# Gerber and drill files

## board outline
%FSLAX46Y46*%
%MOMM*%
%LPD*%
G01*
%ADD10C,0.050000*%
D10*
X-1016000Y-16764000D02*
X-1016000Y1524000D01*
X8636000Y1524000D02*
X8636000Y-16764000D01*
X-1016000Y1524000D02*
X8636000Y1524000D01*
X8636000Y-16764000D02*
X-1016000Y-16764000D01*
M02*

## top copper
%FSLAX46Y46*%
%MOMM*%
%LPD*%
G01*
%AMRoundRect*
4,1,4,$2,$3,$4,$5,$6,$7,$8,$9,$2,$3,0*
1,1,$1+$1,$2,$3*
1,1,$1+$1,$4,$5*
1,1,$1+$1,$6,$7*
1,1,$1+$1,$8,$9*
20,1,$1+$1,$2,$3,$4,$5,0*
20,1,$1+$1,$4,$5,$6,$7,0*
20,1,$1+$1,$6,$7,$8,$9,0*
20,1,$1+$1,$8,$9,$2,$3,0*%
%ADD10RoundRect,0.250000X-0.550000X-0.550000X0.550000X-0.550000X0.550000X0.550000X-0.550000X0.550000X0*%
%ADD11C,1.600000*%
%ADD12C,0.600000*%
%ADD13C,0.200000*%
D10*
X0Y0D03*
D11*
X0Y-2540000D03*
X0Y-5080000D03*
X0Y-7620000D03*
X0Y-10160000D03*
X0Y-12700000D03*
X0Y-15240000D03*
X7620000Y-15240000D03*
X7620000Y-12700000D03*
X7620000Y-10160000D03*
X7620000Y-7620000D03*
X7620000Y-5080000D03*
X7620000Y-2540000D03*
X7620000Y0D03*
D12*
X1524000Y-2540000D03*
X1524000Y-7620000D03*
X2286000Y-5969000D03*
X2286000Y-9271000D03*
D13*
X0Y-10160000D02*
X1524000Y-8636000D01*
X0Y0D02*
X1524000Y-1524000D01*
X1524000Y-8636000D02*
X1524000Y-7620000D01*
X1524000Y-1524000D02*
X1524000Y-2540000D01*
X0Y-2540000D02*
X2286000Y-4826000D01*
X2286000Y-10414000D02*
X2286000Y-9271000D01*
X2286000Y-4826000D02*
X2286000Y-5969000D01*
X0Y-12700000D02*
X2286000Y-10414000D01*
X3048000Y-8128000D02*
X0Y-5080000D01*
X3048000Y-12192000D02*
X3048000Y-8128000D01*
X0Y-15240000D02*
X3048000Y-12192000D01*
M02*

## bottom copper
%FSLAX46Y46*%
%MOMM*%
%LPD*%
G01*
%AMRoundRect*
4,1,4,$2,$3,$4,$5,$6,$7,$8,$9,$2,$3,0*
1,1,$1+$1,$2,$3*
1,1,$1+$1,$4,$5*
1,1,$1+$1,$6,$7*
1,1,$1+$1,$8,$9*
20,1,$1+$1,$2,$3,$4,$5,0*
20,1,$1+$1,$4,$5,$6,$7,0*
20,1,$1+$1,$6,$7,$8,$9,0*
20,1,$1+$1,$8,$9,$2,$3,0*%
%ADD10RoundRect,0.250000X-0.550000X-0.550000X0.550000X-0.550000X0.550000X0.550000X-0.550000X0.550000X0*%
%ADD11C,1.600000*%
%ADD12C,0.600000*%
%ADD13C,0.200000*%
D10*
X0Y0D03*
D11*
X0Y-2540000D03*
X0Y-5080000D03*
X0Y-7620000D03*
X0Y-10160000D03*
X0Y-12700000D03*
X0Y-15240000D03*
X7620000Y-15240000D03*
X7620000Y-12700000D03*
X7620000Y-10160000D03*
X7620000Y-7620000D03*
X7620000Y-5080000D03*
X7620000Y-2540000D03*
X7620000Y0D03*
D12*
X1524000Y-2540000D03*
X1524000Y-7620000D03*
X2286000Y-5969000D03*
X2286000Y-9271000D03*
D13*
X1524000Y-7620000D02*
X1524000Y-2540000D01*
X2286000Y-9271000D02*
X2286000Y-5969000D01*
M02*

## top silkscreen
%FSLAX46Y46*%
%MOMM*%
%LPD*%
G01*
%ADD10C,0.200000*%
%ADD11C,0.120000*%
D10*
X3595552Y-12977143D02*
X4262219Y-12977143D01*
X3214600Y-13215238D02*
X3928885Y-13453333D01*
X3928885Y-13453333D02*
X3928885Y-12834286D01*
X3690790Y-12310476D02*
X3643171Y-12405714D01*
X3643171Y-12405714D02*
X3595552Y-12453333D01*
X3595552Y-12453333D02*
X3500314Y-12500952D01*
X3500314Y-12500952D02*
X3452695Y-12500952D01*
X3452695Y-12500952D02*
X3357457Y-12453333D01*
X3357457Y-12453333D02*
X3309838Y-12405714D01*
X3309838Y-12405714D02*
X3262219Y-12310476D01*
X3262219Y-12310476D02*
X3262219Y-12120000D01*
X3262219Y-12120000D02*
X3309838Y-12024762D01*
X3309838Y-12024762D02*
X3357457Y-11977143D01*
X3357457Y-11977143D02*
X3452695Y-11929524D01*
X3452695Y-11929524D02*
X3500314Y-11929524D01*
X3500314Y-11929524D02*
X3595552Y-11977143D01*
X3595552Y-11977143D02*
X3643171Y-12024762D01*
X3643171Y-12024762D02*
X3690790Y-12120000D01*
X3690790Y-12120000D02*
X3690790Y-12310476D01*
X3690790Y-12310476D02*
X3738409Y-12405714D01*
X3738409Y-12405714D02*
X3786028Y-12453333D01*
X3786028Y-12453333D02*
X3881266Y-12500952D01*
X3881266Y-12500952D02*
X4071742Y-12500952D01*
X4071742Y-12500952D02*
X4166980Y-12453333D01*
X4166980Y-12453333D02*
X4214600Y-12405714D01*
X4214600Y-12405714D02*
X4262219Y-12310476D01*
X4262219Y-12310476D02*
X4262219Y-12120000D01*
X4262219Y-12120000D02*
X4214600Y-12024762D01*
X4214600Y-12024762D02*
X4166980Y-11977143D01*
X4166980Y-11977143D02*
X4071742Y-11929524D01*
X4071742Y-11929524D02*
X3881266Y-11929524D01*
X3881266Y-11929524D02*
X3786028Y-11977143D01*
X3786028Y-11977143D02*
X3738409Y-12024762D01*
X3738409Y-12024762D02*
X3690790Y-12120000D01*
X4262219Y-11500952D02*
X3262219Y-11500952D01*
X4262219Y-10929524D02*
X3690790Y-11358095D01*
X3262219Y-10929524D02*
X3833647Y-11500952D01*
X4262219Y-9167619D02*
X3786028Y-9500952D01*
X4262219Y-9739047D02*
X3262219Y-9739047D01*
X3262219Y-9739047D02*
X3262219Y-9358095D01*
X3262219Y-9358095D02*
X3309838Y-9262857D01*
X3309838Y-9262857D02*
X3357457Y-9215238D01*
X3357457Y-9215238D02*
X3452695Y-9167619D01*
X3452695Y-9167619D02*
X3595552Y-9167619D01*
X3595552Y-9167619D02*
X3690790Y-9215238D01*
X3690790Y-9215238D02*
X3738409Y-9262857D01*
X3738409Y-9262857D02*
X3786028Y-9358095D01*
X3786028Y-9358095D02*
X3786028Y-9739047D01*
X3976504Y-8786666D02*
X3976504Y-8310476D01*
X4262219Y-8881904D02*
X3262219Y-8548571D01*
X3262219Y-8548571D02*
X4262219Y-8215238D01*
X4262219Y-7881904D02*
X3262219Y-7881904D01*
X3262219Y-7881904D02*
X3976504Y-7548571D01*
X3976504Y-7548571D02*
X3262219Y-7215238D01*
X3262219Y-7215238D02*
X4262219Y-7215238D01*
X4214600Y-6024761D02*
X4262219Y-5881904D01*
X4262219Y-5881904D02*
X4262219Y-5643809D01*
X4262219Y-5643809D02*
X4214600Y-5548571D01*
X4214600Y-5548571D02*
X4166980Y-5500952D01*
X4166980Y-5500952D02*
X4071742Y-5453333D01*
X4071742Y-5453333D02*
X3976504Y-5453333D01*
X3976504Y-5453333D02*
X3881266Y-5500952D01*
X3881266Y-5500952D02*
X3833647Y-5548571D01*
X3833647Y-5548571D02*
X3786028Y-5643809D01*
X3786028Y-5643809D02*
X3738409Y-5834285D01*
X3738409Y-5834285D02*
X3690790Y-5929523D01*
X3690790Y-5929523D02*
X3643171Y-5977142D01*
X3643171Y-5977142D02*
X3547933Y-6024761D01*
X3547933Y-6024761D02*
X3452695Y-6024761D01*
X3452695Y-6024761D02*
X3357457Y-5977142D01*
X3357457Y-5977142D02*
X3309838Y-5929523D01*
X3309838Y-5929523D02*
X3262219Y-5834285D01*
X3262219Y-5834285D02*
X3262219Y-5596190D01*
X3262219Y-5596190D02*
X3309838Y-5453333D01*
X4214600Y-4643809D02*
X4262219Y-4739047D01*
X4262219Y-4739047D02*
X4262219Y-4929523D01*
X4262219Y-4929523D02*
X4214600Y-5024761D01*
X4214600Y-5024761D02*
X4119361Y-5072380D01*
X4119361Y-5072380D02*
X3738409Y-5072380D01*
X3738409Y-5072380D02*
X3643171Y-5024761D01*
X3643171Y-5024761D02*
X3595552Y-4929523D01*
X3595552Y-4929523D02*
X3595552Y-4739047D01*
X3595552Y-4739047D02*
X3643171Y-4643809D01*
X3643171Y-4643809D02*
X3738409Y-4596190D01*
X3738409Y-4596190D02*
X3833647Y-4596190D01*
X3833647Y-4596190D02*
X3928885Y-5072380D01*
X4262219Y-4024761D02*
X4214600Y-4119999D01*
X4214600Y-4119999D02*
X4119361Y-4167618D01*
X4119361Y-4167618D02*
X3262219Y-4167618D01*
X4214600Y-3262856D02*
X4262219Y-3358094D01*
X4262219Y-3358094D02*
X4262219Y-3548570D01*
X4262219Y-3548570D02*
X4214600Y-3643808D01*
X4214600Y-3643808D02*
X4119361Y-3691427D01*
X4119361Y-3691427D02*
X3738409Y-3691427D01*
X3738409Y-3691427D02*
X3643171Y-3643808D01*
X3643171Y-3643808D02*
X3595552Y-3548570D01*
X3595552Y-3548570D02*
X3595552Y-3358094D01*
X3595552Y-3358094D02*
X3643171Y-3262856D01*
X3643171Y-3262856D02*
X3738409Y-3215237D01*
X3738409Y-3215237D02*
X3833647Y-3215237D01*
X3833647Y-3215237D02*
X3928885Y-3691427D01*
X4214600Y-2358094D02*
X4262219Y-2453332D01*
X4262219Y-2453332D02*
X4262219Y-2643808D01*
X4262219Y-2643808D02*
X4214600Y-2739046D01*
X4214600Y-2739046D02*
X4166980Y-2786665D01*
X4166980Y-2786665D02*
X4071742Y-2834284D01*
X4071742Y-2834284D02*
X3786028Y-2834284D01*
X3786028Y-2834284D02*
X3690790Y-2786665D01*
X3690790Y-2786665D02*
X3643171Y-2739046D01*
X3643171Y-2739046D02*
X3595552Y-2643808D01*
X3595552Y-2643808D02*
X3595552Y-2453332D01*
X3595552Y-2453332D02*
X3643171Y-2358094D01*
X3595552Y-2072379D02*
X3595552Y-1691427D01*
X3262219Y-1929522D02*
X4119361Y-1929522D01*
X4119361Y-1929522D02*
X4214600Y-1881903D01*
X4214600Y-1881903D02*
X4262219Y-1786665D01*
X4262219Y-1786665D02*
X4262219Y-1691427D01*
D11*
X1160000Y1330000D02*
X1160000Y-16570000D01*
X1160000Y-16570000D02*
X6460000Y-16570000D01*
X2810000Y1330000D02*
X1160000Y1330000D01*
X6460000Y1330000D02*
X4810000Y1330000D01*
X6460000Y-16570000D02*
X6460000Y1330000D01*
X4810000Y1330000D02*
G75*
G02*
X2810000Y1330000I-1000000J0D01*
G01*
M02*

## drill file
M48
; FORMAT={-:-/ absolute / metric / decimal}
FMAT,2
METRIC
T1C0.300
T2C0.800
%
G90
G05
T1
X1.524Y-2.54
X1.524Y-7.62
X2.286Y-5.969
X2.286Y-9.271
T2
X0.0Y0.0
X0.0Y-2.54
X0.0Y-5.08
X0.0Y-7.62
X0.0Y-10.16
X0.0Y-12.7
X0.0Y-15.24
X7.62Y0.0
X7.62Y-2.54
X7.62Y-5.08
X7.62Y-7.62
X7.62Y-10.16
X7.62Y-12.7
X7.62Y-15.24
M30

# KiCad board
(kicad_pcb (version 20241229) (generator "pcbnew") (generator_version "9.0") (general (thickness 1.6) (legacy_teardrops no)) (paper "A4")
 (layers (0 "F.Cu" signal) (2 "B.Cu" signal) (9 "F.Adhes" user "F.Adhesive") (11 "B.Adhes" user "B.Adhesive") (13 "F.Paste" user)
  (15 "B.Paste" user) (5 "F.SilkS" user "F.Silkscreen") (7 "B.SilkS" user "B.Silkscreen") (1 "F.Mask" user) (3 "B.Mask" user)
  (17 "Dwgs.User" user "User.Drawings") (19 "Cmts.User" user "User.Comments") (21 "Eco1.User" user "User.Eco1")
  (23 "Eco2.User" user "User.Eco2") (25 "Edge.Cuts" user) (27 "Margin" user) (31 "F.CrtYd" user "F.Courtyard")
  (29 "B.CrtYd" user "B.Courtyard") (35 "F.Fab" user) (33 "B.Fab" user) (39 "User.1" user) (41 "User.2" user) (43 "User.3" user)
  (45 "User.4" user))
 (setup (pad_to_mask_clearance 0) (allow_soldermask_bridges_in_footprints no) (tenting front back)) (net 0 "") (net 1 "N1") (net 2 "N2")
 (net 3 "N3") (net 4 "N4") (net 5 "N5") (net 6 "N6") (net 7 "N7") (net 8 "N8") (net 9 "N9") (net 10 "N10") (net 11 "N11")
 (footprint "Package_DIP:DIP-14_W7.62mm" (layer "F.Cu") (at 0 0)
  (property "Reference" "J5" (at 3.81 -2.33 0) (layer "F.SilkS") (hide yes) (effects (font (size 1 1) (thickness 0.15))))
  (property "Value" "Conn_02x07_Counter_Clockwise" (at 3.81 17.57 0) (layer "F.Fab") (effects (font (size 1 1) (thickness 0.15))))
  (fp_line (start 1.16 -1.33) (end 1.16 16.57) (stroke (width 0.12) (type solid)) (layer "F.SilkS"))
  (fp_line (start 1.16 16.57) (end 6.46 16.57) (stroke (width 0.12) (type solid)) (layer "F.SilkS"))
  (fp_line (start 2.81 -1.33) (end 1.16 -1.33) (stroke (width 0.12) (type solid)) (layer "F.SilkS"))
  (fp_line (start 6.46 -1.33) (end 4.81 -1.33) (stroke (width 0.12) (type solid)) (layer "F.SilkS"))
  (fp_line (start 6.46 16.57) (end 6.46 -1.33) (stroke (width 0.12) (type solid)) (layer "F.SilkS"))
  (fp_arc (start 4.81 -1.33) (mid 3.81 -0.33) (end 2.81 -1.33) (stroke (width 0.12) (type solid)) (layer "F.SilkS"))
  (pad "1" thru_hole roundrect (at 0 0) (size 1.6 1.6) (drill 0.8) (layers "*.Cu" "*.Mask") (remove_unused_layers no)
   (roundrect_rratio 0.15625) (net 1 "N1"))
  (pad "2" thru_hole circle (at 0 2.54) (size 1.6 1.6) (drill 0.8) (layers "*.Cu" "*.Mask") (remove_unused_layers no) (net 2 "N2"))
  (pad "3" thru_hole circle (at 0 5.08) (size 1.6 1.6) (drill 0.8) (layers "*.Cu" "*.Mask") (remove_unused_layers no) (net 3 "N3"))
  (pad "4" thru_hole circle (at 0 7.62) (size 1.6 1.6) (drill 0.8) (layers "*.Cu" "*.Mask") (remove_unused_layers no) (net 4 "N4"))
  (pad "5" thru_hole circle (at 0 10.16) (size 1.6 1.6) (drill 0.8) (layers "*.Cu" "*.Mask") (remove_unused_layers no) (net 1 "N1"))
  (pad "6" thru_hole circle (at 0 12.7) (size 1.6 1.6) (drill 0.8) (layers "*.Cu" "*.Mask") (remove_unused_layers no) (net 2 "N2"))
  (pad "7" thru_hole circle (at 0 15.24) (size 1.6 1.6) (drill 0.8) (layers "*.Cu" "*.Mask") (remove_unused_layers no) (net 3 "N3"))
  (pad "8" thru_hole circle (at 7.62 15.24) (size 1.6 1.6) (drill 0.8) (layers "*.Cu" "*.Mask") (remove_unused_layers no) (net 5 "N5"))
  (pad "9" thru_hole circle (at 7.62 12.7) (size 1.6 1.6) (drill 0.8) (layers "*.Cu" "*.Mask") (remove_unused_layers no) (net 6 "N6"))
  (pad "10" thru_hole circle (at 7.62 10.16) (size 1.6 1.6) (drill 0.8) (layers "*.Cu" "*.Mask") (remove_unused_layers no) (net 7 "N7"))
  (pad "11" thru_hole circle (at 7.62 7.62) (size 1.6 1.6) (drill 0.8) (layers "*.Cu" "*.Mask") (remove_unused_layers no) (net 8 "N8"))
  (pad "12" thru_hole circle (at 7.62 5.08) (size 1.6 1.6) (drill 0.8) (layers "*.Cu" "*.Mask") (remove_unused_layers no) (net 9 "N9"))
  (pad "13" thru_hole circle (at 7.62 2.54) (size 1.6 1.6) (drill 0.8) (layers "*.Cu" "*.Mask") (remove_unused_layers no) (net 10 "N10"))
  (pad "14" thru_hole circle (at 7.62 0) (size 1.6 1.6) (drill 0.8) (layers "*.Cu" "*.Mask") (remove_unused_layers no) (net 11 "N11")))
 (gr_line (start -1.016 16.764) (end -1.016 -1.524) (stroke (width 0.05) (type default)) (layer "Edge.Cuts"))
 (gr_line (start 8.636 -1.524) (end 8.636 16.764) (stroke (width 0.05) (type default)) (layer "Edge.Cuts"))
 (gr_line (start -1.016 -1.524) (end 8.636 -1.524) (stroke (width 0.05) (type default)) (layer "Edge.Cuts"))
 (gr_line (start 8.636 16.764) (end -1.016 16.764) (stroke (width 0.05) (type default)) (layer "Edge.Cuts"))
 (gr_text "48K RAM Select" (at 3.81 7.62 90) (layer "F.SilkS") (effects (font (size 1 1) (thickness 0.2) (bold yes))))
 (segment (start 0 10.16) (end 1.524 8.636) (width 0.2) (layer "F.Cu") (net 1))
 (segment (start 0 0) (end 1.524 1.524) (width 0.2) (layer "F.Cu") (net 1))
 (segment (start 1.524 8.636) (end 1.524 7.62) (width 0.2) (layer "F.Cu") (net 1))
 (segment (start 1.524 1.524) (end 1.524 2.54) (width 0.2) (layer "F.Cu") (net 1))
 (via (at 1.524 2.54) (size 0.6) (drill 0.3) (layers "F.Cu" "B.Cu") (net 1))
 (via (at 1.524 7.62) (size 0.6) (drill 0.3) (layers "F.Cu" "B.Cu") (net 1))
 (segment (start 1.524 7.62) (end 1.524 2.54) (width 0.2) (layer "B.Cu") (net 1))
 (segment (start 0 2.54) (end 2.286 4.826) (width 0.2) (layer "F.Cu") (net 2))
 (segment (start 2.286 10.414) (end 2.286 9.271) (width 0.2) (layer "F.Cu") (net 2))
 (segment (start 2.286 4.826) (end 2.286 5.969) (width 0.2) (layer "F.Cu") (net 2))
 (segment (start 0 12.7) (end 2.286 10.414) (width 0.2) (layer "F.Cu") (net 2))
 (via (at 2.286 5.969) (size 0.6) (drill 0.3) (layers "F.Cu" "B.Cu") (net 2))
 (via (at 2.286 9.271) (size 0.6) (drill 0.3) (layers "F.Cu" "B.Cu") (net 2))
 (segment (start 2.286 9.271) (end 2.286 5.969) (width 0.2) (layer "B.Cu") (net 2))
 (segment (start 3.048 8.128) (end 0 5.08) (width 0.2) (layer "F.Cu") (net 3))
 (segment (start 3.048 12.192) (end 3.048 8.128) (width 0.2) (layer "F.Cu") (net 3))
 (segment (start 0 15.24) (end 3.048 12.192) (width 0.2) (layer "F.Cu") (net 3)))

